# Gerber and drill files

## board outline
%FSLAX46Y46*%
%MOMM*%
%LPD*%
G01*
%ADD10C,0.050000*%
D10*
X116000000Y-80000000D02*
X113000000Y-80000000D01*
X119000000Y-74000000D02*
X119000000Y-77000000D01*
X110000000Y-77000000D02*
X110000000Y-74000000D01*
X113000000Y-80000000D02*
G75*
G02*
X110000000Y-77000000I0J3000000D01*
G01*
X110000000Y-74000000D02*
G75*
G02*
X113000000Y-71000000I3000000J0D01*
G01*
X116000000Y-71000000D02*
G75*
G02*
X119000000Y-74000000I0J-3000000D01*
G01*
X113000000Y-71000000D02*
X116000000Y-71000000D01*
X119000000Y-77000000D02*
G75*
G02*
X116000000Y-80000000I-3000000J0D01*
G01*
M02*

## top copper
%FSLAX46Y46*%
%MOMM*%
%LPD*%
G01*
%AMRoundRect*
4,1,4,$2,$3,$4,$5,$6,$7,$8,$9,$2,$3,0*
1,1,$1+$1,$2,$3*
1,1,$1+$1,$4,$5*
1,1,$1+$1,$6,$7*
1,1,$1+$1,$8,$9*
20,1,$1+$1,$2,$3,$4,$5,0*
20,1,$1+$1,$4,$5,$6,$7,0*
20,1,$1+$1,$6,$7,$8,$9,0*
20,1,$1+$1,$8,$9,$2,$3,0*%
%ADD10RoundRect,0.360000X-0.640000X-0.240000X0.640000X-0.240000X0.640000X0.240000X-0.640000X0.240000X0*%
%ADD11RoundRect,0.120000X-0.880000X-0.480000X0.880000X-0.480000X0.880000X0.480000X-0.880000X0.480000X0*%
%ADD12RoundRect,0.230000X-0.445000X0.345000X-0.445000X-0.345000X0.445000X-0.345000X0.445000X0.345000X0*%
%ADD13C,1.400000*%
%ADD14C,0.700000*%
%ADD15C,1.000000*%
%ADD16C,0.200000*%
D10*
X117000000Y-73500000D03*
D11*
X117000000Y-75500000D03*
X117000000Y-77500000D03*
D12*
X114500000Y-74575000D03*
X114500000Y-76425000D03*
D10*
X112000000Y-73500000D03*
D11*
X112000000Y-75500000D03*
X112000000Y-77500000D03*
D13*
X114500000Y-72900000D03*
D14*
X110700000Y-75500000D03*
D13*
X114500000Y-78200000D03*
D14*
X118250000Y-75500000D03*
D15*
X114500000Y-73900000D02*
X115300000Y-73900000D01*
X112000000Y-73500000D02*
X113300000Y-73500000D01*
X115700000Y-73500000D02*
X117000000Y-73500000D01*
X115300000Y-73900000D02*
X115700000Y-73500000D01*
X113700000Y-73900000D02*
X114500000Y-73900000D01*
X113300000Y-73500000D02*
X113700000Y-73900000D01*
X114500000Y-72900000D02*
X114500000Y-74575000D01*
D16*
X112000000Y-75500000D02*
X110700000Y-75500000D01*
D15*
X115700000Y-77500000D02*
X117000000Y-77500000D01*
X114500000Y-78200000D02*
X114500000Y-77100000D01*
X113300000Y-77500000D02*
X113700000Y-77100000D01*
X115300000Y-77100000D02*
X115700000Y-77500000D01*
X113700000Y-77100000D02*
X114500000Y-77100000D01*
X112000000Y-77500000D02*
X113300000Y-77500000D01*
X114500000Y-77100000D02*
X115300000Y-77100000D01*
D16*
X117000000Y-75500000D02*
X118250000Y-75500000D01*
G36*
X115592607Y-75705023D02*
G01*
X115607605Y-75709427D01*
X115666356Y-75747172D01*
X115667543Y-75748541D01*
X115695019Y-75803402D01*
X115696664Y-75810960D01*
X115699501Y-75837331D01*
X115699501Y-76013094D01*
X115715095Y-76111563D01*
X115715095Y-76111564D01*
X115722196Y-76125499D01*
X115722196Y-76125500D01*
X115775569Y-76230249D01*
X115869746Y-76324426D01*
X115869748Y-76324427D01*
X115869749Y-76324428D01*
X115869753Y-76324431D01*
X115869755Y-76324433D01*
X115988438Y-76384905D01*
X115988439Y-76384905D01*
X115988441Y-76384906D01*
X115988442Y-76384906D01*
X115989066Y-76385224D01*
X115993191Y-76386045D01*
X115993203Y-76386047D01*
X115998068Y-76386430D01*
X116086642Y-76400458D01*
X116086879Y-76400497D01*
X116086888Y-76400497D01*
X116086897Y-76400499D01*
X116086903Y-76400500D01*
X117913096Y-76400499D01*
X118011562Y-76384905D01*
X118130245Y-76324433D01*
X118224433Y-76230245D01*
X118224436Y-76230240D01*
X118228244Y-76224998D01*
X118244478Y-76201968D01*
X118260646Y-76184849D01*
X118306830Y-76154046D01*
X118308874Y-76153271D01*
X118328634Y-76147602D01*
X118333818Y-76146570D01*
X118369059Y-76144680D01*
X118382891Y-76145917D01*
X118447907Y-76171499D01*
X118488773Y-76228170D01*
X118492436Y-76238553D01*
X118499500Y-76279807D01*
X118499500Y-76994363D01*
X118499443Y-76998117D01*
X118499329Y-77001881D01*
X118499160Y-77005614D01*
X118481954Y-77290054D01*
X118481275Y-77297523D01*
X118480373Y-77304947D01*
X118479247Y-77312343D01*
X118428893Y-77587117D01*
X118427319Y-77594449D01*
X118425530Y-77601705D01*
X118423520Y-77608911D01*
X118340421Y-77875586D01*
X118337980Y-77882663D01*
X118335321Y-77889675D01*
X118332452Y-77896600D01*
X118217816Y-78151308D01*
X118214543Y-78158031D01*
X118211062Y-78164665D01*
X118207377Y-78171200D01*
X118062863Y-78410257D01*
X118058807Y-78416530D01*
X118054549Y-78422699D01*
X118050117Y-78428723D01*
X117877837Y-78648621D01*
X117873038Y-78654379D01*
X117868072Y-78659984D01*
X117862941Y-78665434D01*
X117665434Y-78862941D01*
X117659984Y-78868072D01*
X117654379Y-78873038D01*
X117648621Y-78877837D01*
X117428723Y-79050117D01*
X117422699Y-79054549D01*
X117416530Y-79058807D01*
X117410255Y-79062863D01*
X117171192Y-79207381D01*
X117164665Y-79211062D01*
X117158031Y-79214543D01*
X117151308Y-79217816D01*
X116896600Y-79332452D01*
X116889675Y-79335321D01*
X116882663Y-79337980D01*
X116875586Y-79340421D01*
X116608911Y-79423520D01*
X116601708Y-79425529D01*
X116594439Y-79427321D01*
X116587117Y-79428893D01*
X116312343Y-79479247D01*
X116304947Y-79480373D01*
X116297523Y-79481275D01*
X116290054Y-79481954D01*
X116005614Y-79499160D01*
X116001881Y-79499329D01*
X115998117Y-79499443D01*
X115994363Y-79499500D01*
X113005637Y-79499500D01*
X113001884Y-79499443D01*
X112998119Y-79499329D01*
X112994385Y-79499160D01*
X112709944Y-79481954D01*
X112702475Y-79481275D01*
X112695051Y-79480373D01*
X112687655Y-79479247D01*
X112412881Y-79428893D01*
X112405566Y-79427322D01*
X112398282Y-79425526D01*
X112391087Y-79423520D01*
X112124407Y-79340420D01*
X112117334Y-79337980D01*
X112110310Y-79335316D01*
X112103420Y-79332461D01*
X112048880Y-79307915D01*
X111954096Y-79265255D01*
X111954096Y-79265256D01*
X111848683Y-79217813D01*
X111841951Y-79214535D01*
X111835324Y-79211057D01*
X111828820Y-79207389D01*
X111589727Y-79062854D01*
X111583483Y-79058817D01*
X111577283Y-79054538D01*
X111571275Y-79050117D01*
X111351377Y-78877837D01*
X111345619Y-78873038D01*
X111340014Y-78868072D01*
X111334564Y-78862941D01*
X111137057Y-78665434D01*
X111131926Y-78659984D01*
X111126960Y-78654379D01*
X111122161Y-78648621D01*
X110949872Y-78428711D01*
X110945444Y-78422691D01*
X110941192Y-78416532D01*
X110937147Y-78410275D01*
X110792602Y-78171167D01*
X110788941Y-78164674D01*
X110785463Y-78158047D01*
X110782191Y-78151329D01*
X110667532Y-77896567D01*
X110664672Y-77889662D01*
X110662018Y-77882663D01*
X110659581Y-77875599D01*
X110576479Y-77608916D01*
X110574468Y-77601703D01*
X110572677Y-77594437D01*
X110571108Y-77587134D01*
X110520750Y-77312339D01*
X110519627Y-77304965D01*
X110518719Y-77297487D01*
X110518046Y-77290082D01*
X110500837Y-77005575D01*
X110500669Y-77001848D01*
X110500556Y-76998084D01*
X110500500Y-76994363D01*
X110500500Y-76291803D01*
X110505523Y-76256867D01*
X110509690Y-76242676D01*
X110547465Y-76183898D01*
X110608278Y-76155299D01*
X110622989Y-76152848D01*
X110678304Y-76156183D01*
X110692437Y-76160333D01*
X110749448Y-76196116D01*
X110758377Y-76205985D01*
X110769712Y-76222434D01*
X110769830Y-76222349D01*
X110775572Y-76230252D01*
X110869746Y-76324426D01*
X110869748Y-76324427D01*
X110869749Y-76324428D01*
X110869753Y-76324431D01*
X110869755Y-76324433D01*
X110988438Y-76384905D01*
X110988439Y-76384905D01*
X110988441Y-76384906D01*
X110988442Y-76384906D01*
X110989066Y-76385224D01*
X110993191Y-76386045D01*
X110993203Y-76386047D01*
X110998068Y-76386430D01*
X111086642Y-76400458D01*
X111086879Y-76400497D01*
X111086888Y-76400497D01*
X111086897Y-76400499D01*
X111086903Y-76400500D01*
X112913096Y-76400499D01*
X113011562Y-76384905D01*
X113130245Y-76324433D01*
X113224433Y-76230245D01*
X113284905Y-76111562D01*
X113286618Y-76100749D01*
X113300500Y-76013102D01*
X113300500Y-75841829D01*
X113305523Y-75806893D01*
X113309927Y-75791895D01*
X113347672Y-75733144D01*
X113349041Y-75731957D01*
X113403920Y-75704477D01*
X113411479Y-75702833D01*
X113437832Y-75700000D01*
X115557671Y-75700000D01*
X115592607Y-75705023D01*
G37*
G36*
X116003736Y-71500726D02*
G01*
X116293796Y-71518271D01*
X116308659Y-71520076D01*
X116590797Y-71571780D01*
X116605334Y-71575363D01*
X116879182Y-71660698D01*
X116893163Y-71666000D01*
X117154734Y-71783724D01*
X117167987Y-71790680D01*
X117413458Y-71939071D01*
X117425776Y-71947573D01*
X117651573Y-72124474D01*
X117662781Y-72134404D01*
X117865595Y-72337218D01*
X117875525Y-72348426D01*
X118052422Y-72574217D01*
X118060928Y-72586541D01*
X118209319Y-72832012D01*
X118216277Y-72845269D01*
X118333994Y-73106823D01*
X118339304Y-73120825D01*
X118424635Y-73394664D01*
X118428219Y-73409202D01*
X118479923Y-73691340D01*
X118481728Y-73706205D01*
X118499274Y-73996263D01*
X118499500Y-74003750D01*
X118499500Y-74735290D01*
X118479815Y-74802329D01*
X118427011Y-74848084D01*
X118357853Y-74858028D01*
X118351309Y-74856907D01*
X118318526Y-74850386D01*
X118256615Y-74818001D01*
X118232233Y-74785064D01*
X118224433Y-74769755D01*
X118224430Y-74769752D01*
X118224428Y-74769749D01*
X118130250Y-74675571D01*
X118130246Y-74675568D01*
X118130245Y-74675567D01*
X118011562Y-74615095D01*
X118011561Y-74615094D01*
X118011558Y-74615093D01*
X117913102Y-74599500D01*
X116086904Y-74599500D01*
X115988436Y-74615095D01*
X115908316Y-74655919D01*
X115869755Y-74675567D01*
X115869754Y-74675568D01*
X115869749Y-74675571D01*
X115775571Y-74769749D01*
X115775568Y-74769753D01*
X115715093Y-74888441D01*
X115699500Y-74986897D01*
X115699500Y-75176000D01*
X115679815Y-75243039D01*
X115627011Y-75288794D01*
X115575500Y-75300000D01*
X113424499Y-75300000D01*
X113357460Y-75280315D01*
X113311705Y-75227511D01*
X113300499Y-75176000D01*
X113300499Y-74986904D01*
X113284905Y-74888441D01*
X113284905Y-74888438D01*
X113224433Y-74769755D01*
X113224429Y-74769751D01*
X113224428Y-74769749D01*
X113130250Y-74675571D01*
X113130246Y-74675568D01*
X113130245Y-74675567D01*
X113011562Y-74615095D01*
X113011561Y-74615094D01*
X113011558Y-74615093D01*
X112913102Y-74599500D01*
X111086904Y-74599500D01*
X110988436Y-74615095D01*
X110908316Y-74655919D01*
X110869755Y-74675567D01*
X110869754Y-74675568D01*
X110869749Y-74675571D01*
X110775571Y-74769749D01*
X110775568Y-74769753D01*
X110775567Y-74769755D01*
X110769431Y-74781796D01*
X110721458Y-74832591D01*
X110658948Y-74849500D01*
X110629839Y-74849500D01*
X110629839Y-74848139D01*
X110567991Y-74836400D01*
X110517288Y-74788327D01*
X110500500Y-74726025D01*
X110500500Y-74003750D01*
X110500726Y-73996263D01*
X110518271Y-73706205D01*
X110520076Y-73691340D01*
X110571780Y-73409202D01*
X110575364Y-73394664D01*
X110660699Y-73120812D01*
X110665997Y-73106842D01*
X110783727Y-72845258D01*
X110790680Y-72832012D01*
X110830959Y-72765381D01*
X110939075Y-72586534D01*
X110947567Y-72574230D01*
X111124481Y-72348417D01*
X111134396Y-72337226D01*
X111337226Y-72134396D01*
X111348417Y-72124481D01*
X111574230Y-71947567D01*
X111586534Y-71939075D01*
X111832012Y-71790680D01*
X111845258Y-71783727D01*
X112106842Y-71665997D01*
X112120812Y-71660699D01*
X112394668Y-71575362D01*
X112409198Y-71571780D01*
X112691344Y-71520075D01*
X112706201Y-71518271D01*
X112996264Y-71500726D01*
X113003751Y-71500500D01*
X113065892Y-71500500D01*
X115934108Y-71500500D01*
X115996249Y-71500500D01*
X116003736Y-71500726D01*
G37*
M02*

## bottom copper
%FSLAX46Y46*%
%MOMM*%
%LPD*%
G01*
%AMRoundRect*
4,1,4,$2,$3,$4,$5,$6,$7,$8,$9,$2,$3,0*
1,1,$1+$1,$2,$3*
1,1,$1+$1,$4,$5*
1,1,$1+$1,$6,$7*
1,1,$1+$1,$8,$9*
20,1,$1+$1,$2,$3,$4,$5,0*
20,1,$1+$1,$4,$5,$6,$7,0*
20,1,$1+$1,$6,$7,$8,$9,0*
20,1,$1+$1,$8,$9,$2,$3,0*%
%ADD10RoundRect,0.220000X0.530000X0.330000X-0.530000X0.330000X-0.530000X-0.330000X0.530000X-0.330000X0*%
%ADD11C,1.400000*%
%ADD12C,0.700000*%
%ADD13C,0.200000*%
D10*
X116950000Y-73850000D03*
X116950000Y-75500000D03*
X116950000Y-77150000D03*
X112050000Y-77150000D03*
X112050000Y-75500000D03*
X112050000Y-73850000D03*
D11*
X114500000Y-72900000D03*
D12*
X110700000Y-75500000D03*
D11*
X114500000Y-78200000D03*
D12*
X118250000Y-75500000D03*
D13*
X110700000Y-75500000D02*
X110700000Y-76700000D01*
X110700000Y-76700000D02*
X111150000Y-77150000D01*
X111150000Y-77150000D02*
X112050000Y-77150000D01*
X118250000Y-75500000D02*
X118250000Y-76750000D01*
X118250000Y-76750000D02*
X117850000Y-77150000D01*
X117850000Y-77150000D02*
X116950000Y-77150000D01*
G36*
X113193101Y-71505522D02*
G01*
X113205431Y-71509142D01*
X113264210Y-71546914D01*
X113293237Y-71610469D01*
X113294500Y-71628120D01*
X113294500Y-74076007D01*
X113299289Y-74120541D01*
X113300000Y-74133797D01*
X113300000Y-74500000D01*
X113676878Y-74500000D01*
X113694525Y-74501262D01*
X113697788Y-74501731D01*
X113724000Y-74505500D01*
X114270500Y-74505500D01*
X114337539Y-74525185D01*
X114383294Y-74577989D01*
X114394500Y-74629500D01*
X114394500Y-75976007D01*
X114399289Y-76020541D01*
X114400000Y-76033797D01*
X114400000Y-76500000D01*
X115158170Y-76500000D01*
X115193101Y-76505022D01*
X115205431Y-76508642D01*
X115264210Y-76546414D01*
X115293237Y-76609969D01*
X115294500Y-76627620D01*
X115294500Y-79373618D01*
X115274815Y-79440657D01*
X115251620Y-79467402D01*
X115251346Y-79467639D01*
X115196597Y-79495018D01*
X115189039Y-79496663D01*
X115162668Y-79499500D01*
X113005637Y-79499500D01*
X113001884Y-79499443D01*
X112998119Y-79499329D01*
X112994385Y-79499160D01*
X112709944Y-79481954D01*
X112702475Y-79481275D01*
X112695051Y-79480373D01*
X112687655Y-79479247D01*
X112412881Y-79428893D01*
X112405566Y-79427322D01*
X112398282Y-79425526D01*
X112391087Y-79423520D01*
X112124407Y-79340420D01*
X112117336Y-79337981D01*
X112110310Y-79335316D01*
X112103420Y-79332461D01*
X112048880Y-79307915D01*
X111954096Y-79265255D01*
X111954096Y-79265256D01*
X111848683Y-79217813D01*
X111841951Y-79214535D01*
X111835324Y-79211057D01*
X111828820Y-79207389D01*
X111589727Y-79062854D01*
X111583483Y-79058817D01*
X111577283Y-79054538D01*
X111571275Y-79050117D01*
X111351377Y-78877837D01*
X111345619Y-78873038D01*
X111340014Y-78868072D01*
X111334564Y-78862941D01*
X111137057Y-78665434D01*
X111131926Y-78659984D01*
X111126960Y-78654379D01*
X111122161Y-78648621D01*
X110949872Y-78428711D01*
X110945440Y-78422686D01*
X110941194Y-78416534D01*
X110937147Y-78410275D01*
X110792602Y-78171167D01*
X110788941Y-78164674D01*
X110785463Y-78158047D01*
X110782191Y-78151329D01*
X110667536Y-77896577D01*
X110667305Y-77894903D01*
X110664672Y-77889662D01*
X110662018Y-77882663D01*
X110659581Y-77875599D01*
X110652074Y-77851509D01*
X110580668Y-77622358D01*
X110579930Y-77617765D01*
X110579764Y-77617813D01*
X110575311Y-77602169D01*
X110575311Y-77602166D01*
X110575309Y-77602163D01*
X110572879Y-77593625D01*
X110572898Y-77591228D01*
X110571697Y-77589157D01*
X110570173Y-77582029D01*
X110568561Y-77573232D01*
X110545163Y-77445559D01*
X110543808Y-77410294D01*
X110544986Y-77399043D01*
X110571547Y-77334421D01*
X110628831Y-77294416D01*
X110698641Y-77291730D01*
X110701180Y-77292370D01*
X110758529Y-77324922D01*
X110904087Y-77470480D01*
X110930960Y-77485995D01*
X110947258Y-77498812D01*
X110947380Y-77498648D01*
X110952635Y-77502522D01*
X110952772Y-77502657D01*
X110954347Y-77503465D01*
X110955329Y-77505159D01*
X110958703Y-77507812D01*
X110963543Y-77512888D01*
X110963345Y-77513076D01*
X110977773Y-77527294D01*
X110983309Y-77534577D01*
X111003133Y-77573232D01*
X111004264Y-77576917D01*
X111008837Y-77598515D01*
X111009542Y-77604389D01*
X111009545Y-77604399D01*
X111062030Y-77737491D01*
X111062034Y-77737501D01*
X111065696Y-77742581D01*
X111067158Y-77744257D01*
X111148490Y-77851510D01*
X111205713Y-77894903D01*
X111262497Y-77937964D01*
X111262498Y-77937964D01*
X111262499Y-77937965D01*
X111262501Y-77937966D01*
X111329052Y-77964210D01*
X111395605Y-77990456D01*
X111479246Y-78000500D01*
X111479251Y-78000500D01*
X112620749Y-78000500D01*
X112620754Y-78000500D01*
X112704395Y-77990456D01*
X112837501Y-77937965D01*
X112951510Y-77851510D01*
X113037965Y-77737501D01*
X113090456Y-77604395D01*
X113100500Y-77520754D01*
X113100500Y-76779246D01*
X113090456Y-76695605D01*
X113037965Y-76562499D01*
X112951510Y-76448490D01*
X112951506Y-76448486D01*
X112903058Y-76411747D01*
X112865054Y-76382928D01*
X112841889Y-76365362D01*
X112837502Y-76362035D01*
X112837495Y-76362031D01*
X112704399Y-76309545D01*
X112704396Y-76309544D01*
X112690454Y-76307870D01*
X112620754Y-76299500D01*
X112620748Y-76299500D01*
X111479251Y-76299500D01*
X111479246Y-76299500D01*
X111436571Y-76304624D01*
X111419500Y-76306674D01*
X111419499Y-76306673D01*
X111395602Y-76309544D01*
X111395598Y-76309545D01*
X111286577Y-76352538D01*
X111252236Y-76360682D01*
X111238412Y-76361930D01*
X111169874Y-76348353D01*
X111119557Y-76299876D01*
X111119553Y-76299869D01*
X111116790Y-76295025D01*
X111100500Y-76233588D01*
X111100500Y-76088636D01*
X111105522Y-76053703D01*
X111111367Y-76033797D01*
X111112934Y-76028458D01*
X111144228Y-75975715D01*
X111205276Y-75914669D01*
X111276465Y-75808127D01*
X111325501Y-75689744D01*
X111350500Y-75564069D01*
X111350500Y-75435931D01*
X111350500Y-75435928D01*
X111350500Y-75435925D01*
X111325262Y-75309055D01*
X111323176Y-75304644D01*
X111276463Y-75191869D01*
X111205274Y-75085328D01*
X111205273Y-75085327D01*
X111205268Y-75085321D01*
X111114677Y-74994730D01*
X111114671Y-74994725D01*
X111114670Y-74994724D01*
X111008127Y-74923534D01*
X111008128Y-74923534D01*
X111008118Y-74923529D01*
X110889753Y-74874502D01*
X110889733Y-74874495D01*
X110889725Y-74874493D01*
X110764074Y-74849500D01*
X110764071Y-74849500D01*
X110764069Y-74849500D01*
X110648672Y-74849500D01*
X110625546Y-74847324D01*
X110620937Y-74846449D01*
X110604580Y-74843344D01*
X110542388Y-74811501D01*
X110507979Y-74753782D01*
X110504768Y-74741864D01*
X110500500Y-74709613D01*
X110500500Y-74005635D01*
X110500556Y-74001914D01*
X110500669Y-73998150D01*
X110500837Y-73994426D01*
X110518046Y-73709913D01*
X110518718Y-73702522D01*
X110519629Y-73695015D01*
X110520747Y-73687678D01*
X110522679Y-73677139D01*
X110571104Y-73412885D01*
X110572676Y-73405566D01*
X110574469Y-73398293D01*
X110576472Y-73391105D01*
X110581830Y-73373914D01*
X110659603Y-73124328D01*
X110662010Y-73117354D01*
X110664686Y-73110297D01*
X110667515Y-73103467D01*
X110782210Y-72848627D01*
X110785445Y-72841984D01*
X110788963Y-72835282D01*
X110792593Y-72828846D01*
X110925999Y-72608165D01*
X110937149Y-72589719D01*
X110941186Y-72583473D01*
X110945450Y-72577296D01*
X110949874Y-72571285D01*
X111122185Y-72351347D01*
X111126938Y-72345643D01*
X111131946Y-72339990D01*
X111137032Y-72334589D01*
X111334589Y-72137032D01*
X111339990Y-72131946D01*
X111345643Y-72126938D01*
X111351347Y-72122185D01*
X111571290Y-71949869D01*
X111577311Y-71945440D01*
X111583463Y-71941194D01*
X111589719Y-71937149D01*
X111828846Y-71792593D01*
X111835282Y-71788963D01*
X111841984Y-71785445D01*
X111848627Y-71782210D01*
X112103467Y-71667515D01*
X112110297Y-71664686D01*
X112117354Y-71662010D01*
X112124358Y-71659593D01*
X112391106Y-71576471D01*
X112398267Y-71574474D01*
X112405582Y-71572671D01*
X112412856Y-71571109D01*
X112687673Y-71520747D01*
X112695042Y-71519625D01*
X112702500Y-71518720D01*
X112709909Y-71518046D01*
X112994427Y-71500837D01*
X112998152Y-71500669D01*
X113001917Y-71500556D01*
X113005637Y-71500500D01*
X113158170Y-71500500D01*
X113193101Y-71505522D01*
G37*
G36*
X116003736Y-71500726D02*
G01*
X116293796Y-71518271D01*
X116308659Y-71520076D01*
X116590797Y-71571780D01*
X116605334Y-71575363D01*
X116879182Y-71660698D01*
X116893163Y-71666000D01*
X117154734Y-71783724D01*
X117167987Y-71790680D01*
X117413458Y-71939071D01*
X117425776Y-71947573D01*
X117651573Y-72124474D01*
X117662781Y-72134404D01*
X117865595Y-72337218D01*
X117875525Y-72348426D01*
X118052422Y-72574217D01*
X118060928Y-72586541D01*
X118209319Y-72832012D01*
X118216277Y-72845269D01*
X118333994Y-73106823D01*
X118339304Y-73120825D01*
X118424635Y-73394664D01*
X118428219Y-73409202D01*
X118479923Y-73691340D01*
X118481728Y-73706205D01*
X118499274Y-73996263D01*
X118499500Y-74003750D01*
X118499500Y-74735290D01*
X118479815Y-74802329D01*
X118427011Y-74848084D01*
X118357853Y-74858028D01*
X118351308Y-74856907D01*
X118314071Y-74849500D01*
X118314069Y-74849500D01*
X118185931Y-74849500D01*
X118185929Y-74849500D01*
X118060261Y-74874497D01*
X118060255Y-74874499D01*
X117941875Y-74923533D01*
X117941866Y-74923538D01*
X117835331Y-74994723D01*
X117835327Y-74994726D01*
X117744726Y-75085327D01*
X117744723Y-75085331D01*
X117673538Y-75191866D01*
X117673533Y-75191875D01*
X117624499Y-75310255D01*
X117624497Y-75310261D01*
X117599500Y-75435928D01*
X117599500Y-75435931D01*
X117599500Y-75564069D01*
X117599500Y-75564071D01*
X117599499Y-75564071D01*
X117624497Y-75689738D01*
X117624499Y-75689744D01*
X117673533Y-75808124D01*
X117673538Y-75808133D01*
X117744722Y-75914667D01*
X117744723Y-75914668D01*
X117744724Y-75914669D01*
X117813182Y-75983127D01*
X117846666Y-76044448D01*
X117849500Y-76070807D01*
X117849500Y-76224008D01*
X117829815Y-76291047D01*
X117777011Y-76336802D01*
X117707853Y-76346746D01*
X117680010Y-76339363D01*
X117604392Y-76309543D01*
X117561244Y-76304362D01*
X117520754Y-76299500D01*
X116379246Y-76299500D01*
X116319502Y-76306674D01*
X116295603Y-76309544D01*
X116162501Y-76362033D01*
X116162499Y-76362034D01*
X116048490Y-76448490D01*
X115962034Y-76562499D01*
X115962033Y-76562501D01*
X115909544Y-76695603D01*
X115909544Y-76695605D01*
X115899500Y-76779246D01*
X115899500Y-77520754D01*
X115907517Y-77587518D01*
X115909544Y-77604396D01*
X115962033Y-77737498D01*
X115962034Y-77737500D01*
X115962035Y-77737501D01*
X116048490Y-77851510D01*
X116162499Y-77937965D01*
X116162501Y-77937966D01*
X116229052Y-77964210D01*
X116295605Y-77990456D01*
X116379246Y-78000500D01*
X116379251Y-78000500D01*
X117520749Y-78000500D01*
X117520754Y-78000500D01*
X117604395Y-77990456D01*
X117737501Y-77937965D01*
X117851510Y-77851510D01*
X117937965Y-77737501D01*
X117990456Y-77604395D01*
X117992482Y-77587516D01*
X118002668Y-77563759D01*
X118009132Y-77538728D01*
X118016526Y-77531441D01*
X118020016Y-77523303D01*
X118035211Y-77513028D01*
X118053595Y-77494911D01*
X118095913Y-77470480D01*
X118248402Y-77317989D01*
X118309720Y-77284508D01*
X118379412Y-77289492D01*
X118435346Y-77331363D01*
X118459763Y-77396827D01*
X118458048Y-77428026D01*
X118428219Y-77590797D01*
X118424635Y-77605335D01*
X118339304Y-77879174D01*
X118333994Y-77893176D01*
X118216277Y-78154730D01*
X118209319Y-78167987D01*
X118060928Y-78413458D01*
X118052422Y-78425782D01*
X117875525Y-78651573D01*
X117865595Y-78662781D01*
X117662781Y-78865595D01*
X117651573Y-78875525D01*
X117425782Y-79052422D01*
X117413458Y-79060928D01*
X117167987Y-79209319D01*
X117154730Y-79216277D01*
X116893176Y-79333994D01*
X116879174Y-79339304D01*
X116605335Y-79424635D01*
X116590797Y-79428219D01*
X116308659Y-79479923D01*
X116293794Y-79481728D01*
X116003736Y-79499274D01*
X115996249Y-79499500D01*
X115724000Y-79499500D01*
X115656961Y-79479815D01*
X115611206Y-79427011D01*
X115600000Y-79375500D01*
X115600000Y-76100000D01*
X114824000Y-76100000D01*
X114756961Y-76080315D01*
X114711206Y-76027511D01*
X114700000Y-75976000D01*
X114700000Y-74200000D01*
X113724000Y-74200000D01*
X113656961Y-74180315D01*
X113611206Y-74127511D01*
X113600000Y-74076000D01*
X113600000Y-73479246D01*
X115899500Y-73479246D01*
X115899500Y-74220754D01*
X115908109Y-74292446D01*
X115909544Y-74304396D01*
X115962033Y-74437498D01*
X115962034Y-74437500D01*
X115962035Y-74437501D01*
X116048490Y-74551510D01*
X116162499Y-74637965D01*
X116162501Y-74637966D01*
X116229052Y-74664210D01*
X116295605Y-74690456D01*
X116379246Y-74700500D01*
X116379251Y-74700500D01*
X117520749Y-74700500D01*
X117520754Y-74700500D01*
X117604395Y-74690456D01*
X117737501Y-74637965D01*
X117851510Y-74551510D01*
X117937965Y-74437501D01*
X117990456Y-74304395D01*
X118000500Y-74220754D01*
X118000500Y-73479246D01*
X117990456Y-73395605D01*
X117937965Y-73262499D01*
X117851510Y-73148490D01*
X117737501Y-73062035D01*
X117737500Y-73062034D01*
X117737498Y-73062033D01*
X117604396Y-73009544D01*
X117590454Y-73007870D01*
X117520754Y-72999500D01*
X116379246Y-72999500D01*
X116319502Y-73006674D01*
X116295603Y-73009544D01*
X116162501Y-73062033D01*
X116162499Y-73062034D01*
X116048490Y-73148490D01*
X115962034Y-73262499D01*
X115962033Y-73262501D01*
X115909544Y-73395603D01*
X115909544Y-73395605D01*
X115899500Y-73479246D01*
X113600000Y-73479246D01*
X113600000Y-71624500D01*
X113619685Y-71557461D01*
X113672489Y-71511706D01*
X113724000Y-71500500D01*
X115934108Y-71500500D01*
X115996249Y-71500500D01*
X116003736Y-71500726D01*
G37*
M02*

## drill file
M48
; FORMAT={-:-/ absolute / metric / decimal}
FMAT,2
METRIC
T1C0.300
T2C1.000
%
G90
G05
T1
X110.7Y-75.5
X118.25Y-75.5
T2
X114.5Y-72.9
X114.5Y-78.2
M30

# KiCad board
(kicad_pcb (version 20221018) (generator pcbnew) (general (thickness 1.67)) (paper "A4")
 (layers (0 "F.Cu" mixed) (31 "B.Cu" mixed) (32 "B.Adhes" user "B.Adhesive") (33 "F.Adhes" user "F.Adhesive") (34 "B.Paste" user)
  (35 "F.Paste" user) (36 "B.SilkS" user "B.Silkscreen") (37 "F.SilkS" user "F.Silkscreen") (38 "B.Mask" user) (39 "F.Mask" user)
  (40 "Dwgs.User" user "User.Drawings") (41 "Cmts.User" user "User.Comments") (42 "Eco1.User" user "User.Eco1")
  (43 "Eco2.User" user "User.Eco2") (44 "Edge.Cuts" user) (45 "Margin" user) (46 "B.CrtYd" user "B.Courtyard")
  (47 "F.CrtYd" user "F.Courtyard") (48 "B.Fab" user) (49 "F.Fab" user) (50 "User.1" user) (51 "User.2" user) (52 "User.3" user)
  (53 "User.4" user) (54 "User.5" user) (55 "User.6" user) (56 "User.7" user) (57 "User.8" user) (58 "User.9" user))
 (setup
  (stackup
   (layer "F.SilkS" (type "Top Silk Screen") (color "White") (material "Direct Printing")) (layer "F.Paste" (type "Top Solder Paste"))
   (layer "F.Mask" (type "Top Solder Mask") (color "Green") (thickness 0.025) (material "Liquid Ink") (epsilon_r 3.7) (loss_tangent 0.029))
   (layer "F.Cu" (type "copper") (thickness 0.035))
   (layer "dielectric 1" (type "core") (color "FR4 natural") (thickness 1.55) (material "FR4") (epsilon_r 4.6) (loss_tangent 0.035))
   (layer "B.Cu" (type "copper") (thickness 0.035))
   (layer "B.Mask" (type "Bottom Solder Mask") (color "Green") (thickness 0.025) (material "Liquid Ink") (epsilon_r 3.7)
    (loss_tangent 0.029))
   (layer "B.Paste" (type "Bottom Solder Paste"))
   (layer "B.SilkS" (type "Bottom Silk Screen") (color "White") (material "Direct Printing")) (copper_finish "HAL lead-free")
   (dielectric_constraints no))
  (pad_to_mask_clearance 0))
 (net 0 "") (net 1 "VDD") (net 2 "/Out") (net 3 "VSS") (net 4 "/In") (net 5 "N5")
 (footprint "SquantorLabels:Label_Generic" (layer "F.Cu") (at 138.1 91.5)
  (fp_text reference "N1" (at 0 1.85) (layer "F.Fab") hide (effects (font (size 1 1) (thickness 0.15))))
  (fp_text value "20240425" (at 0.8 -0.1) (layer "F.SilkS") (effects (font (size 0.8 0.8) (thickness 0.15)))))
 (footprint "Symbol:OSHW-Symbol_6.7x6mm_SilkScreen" (layer "F.Cu") (at 138.7 87.6)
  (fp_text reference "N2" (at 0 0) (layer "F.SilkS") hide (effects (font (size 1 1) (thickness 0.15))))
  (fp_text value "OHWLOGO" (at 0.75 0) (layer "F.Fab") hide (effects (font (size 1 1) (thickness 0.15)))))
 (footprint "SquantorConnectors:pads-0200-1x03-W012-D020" (layer "F.Cu") (at 117 75.5)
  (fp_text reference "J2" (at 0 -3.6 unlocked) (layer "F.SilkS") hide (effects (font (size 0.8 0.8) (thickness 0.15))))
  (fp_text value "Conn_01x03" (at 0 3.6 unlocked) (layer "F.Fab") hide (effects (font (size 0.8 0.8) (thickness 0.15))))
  (pad "1" smd roundrect (at 0 -2) (size 2 1.2) (layers "F.Cu" "F.Paste" "F.Mask") (roundrect_rratio 0.3) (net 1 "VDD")
   (thermal_bridge_angle 45))
  (pad "2" smd roundrect (at 0 0) (size 2 1.2) (layers "F.Cu" "F.Paste" "F.Mask") (roundrect_rratio 0.1) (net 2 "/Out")
   (thermal_bridge_angle 45))
  (pad "3" smd roundrect (at 0 2) (size 2 1.2) (layers "F.Cu" "F.Paste" "F.Mask") (roundrect_rratio 0.1) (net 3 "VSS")
   (thermal_bridge_angle 45)))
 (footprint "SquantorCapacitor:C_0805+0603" (layer "F.Cu") (at 114.5 75.5 -90)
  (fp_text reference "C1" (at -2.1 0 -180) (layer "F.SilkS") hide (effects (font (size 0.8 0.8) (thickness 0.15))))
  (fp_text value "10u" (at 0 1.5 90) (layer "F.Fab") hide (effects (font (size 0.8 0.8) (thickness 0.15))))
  (pad "1" smd roundrect (at -0.925 0 270) (size 1.15 1.35) (layers "F.Cu" "F.Paste" "F.Mask") (roundrect_rratio 0.2) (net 1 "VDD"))
  (pad "2" smd roundrect (at 0.925 0 270) (size 1.15 1.35) (layers "F.Cu" "F.Paste" "F.Mask") (roundrect_rratio 0.2) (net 3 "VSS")))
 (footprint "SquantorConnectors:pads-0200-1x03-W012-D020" (layer "F.Cu") (at 112 75.5)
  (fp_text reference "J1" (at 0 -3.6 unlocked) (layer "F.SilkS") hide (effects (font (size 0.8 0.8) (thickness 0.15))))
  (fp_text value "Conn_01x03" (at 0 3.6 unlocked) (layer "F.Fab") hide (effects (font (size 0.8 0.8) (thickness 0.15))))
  (pad "1" smd roundrect (at 0 -2) (size 2 1.2) (layers "F.Cu" "F.Paste" "F.Mask") (roundrect_rratio 0.3) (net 1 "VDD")
   (thermal_bridge_angle 45))
  (pad "2" smd roundrect (at 0 0) (size 2 1.2) (layers "F.Cu" "F.Paste" "F.Mask") (roundrect_rratio 0.1) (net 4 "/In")
   (thermal_bridge_angle 45))
  (pad "3" smd roundrect (at 0 2) (size 2 1.2) (layers "F.Cu" "F.Paste" "F.Mask") (roundrect_rratio 0.1) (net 3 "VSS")
   (thermal_bridge_angle 45)))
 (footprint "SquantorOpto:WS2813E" (layer "B.Cu") (at 114.5 75.5 180)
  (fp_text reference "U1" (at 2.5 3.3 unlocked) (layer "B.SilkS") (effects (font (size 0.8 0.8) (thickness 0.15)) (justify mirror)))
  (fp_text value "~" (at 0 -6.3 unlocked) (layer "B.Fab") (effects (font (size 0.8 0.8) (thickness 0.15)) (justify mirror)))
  (pad "1" smd roundrect (at -2.45 1.65 180) (size 1.5 1.1) (layers "B.Cu" "B.Paste" "B.Mask") (roundrect_rratio 0.2) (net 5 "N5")
   (thermal_bridge_angle 45))
  (pad "2" smd roundrect (at -2.45 0 180) (size 1.5 1.1) (layers "B.Cu" "B.Paste" "B.Mask") (roundrect_rratio 0.2) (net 1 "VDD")
   (thermal_bridge_angle 45))
  (pad "3" smd roundrect (at -2.45 -1.65 180) (size 1.5 1.1) (layers "B.Cu" "B.Paste" "B.Mask") (roundrect_rratio 0.2) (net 2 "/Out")
   (thermal_bridge_angle 45))
  (pad "4" smd roundrect (at 2.45 -1.65 180) (size 1.5 1.1) (layers "B.Cu" "B.Paste" "B.Mask") (roundrect_rratio 0.2) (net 4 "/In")
   (thermal_bridge_angle 45))
  (pad "5" smd roundrect (at 2.45 0 180) (size 1.5 1.1) (layers "B.Cu" "B.Paste" "B.Mask") (roundrect_rratio 0.2) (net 3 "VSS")
   (thermal_bridge_angle 45))
  (pad "6" smd roundrect (at 2.45 1.65 180) (size 1.5 1.1) (layers "B.Cu" "B.Paste" "B.Mask") (roundrect_rratio 0.2) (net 3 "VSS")
   (thermal_bridge_angle 45)))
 (gr_line (start 116 80) (end 113 80) (stroke (width 0.05) (type default)) (layer "Edge.Cuts"))
 (gr_line (start 119 74) (end 119 77) (stroke (width 0.05) (type default)) (layer "Edge.Cuts"))
 (gr_line (start 110 77) (end 110 74) (stroke (width 0.05) (type default)) (layer "Edge.Cuts"))
 (gr_arc (start 113 80) (mid 110.87868 79.12132) (end 110 77) (stroke (width 0.05) (type default)) (layer "Edge.Cuts"))
 (gr_arc (start 110 74) (mid 110.87868 71.87868) (end 113 71) (stroke (width 0.05) (type default)) (layer "Edge.Cuts"))
 (gr_arc (start 116 71) (mid 118.12132 71.87868) (end 119 74) (stroke (width 0.05) (type default)) (layer "Edge.Cuts"))
 (gr_line (start 113 71) (end 116 71) (stroke (width 0.05) (type default)) (layer "Edge.Cuts"))
 (gr_arc (start 119 77) (mid 118.12132 79.12132) (end 116 80) (stroke (width 0.05) (type default)) (layer "Edge.Cuts"))
 (segment (start 114.5 73.9) (end 115.3 73.9) (width 1) (layer "F.Cu") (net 1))
 (segment (start 112 73.5) (end 113.3 73.5) (width 1) (layer "F.Cu") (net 1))
 (segment (start 115.7 73.5) (end 117 73.5) (width 1) (layer "F.Cu") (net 1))
 (segment (start 115.3 73.9) (end 115.7 73.5) (width 1) (layer "F.Cu") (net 1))
 (segment (start 113.7 73.9) (end 114.5 73.9) (width 1) (layer "F.Cu") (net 1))
 (segment (start 113.3 73.5) (end 113.7 73.9) (width 1) (layer "F.Cu") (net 1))
 (segment (start 114.5 72.9) (end 114.5 74.575) (width 1) (layer "F.Cu") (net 1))
 (via (at 114.5 72.9) (size 1.4) (drill 1) (layers "F.Cu" "B.Cu") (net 1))
 (segment (start 112 75.5) (end 110.7 75.5) (width 0.2) (layer "F.Cu") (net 4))
 (via (at 110.7 75.5) (size 0.7) (drill 0.3) (layers "F.Cu" "B.Cu") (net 4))
 (segment (start 110.7 75.5) (end 110.7 76.7) (width 0.2) (layer "B.Cu") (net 4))
 (segment (start 110.7 76.7) (end 111.15 77.15) (width 0.2) (layer "B.Cu") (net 4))
 (segment (start 111.15 77.15) (end 112.05 77.15) (width 0.2) (layer "B.Cu") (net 4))
 (segment (start 115.7 77.5) (end 117 77.5) (width 1) (layer "F.Cu") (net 3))
 (segment (start 114.5 78.2) (end 114.5 77.1) (width 1) (layer "F.Cu") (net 3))
 (segment (start 113.3 77.5) (end 113.7 77.1) (width 1) (layer "F.Cu") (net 3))
 (segment (start 115.3 77.1) (end 115.7 77.5) (width 1) (layer "F.Cu") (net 3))
 (segment (start 113.7 77.1) (end 114.5 77.1) (width 1) (layer "F.Cu") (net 3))
 (segment (start 112 77.5) (end 113.3 77.5) (width 1) (layer "F.Cu") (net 3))
 (segment (start 114.5 77.1) (end 115.3 77.1) (width 1) (layer "F.Cu") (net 3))
 (via (at 114.5 78.2) (size 1.4) (drill 1) (layers "F.Cu" "B.Cu") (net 3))
 (segment (start 117 75.5) (end 118.25 75.5) (width 0.2) (layer "F.Cu") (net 2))
 (via (at 118.25 75.5) (size 0.7) (drill 0.3) (layers "F.Cu" "B.Cu") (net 2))
 (segment (start 118.25 75.5) (end 118.25 76.75) (width 0.2) (layer "B.Cu") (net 2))
 (segment (start 118.25 76.75) (end 117.85 77.15) (width 0.2) (layer "B.Cu") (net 2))
 (segment (start 117.85 77.15) (end 116.95 77.15) (width 0.2) (layer "B.Cu") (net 2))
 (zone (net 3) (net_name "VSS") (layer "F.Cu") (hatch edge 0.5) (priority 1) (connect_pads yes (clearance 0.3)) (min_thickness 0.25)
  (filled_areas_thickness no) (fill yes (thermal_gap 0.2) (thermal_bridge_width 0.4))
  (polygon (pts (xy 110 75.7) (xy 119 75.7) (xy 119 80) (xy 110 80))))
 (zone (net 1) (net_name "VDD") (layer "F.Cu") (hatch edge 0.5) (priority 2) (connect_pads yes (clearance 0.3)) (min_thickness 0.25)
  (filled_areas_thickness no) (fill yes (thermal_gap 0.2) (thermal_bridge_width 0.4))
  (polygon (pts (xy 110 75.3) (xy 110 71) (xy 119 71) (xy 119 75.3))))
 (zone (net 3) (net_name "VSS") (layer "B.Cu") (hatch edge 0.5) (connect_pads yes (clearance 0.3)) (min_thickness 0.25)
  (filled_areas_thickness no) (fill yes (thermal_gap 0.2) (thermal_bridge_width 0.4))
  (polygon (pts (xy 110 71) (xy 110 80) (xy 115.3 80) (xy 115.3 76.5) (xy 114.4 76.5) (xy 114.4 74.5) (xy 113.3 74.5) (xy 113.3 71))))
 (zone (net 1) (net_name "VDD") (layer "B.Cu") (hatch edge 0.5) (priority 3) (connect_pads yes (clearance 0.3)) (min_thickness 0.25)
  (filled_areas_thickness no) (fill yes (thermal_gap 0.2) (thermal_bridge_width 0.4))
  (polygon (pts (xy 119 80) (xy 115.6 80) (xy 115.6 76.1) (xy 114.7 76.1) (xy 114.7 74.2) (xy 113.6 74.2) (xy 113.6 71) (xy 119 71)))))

